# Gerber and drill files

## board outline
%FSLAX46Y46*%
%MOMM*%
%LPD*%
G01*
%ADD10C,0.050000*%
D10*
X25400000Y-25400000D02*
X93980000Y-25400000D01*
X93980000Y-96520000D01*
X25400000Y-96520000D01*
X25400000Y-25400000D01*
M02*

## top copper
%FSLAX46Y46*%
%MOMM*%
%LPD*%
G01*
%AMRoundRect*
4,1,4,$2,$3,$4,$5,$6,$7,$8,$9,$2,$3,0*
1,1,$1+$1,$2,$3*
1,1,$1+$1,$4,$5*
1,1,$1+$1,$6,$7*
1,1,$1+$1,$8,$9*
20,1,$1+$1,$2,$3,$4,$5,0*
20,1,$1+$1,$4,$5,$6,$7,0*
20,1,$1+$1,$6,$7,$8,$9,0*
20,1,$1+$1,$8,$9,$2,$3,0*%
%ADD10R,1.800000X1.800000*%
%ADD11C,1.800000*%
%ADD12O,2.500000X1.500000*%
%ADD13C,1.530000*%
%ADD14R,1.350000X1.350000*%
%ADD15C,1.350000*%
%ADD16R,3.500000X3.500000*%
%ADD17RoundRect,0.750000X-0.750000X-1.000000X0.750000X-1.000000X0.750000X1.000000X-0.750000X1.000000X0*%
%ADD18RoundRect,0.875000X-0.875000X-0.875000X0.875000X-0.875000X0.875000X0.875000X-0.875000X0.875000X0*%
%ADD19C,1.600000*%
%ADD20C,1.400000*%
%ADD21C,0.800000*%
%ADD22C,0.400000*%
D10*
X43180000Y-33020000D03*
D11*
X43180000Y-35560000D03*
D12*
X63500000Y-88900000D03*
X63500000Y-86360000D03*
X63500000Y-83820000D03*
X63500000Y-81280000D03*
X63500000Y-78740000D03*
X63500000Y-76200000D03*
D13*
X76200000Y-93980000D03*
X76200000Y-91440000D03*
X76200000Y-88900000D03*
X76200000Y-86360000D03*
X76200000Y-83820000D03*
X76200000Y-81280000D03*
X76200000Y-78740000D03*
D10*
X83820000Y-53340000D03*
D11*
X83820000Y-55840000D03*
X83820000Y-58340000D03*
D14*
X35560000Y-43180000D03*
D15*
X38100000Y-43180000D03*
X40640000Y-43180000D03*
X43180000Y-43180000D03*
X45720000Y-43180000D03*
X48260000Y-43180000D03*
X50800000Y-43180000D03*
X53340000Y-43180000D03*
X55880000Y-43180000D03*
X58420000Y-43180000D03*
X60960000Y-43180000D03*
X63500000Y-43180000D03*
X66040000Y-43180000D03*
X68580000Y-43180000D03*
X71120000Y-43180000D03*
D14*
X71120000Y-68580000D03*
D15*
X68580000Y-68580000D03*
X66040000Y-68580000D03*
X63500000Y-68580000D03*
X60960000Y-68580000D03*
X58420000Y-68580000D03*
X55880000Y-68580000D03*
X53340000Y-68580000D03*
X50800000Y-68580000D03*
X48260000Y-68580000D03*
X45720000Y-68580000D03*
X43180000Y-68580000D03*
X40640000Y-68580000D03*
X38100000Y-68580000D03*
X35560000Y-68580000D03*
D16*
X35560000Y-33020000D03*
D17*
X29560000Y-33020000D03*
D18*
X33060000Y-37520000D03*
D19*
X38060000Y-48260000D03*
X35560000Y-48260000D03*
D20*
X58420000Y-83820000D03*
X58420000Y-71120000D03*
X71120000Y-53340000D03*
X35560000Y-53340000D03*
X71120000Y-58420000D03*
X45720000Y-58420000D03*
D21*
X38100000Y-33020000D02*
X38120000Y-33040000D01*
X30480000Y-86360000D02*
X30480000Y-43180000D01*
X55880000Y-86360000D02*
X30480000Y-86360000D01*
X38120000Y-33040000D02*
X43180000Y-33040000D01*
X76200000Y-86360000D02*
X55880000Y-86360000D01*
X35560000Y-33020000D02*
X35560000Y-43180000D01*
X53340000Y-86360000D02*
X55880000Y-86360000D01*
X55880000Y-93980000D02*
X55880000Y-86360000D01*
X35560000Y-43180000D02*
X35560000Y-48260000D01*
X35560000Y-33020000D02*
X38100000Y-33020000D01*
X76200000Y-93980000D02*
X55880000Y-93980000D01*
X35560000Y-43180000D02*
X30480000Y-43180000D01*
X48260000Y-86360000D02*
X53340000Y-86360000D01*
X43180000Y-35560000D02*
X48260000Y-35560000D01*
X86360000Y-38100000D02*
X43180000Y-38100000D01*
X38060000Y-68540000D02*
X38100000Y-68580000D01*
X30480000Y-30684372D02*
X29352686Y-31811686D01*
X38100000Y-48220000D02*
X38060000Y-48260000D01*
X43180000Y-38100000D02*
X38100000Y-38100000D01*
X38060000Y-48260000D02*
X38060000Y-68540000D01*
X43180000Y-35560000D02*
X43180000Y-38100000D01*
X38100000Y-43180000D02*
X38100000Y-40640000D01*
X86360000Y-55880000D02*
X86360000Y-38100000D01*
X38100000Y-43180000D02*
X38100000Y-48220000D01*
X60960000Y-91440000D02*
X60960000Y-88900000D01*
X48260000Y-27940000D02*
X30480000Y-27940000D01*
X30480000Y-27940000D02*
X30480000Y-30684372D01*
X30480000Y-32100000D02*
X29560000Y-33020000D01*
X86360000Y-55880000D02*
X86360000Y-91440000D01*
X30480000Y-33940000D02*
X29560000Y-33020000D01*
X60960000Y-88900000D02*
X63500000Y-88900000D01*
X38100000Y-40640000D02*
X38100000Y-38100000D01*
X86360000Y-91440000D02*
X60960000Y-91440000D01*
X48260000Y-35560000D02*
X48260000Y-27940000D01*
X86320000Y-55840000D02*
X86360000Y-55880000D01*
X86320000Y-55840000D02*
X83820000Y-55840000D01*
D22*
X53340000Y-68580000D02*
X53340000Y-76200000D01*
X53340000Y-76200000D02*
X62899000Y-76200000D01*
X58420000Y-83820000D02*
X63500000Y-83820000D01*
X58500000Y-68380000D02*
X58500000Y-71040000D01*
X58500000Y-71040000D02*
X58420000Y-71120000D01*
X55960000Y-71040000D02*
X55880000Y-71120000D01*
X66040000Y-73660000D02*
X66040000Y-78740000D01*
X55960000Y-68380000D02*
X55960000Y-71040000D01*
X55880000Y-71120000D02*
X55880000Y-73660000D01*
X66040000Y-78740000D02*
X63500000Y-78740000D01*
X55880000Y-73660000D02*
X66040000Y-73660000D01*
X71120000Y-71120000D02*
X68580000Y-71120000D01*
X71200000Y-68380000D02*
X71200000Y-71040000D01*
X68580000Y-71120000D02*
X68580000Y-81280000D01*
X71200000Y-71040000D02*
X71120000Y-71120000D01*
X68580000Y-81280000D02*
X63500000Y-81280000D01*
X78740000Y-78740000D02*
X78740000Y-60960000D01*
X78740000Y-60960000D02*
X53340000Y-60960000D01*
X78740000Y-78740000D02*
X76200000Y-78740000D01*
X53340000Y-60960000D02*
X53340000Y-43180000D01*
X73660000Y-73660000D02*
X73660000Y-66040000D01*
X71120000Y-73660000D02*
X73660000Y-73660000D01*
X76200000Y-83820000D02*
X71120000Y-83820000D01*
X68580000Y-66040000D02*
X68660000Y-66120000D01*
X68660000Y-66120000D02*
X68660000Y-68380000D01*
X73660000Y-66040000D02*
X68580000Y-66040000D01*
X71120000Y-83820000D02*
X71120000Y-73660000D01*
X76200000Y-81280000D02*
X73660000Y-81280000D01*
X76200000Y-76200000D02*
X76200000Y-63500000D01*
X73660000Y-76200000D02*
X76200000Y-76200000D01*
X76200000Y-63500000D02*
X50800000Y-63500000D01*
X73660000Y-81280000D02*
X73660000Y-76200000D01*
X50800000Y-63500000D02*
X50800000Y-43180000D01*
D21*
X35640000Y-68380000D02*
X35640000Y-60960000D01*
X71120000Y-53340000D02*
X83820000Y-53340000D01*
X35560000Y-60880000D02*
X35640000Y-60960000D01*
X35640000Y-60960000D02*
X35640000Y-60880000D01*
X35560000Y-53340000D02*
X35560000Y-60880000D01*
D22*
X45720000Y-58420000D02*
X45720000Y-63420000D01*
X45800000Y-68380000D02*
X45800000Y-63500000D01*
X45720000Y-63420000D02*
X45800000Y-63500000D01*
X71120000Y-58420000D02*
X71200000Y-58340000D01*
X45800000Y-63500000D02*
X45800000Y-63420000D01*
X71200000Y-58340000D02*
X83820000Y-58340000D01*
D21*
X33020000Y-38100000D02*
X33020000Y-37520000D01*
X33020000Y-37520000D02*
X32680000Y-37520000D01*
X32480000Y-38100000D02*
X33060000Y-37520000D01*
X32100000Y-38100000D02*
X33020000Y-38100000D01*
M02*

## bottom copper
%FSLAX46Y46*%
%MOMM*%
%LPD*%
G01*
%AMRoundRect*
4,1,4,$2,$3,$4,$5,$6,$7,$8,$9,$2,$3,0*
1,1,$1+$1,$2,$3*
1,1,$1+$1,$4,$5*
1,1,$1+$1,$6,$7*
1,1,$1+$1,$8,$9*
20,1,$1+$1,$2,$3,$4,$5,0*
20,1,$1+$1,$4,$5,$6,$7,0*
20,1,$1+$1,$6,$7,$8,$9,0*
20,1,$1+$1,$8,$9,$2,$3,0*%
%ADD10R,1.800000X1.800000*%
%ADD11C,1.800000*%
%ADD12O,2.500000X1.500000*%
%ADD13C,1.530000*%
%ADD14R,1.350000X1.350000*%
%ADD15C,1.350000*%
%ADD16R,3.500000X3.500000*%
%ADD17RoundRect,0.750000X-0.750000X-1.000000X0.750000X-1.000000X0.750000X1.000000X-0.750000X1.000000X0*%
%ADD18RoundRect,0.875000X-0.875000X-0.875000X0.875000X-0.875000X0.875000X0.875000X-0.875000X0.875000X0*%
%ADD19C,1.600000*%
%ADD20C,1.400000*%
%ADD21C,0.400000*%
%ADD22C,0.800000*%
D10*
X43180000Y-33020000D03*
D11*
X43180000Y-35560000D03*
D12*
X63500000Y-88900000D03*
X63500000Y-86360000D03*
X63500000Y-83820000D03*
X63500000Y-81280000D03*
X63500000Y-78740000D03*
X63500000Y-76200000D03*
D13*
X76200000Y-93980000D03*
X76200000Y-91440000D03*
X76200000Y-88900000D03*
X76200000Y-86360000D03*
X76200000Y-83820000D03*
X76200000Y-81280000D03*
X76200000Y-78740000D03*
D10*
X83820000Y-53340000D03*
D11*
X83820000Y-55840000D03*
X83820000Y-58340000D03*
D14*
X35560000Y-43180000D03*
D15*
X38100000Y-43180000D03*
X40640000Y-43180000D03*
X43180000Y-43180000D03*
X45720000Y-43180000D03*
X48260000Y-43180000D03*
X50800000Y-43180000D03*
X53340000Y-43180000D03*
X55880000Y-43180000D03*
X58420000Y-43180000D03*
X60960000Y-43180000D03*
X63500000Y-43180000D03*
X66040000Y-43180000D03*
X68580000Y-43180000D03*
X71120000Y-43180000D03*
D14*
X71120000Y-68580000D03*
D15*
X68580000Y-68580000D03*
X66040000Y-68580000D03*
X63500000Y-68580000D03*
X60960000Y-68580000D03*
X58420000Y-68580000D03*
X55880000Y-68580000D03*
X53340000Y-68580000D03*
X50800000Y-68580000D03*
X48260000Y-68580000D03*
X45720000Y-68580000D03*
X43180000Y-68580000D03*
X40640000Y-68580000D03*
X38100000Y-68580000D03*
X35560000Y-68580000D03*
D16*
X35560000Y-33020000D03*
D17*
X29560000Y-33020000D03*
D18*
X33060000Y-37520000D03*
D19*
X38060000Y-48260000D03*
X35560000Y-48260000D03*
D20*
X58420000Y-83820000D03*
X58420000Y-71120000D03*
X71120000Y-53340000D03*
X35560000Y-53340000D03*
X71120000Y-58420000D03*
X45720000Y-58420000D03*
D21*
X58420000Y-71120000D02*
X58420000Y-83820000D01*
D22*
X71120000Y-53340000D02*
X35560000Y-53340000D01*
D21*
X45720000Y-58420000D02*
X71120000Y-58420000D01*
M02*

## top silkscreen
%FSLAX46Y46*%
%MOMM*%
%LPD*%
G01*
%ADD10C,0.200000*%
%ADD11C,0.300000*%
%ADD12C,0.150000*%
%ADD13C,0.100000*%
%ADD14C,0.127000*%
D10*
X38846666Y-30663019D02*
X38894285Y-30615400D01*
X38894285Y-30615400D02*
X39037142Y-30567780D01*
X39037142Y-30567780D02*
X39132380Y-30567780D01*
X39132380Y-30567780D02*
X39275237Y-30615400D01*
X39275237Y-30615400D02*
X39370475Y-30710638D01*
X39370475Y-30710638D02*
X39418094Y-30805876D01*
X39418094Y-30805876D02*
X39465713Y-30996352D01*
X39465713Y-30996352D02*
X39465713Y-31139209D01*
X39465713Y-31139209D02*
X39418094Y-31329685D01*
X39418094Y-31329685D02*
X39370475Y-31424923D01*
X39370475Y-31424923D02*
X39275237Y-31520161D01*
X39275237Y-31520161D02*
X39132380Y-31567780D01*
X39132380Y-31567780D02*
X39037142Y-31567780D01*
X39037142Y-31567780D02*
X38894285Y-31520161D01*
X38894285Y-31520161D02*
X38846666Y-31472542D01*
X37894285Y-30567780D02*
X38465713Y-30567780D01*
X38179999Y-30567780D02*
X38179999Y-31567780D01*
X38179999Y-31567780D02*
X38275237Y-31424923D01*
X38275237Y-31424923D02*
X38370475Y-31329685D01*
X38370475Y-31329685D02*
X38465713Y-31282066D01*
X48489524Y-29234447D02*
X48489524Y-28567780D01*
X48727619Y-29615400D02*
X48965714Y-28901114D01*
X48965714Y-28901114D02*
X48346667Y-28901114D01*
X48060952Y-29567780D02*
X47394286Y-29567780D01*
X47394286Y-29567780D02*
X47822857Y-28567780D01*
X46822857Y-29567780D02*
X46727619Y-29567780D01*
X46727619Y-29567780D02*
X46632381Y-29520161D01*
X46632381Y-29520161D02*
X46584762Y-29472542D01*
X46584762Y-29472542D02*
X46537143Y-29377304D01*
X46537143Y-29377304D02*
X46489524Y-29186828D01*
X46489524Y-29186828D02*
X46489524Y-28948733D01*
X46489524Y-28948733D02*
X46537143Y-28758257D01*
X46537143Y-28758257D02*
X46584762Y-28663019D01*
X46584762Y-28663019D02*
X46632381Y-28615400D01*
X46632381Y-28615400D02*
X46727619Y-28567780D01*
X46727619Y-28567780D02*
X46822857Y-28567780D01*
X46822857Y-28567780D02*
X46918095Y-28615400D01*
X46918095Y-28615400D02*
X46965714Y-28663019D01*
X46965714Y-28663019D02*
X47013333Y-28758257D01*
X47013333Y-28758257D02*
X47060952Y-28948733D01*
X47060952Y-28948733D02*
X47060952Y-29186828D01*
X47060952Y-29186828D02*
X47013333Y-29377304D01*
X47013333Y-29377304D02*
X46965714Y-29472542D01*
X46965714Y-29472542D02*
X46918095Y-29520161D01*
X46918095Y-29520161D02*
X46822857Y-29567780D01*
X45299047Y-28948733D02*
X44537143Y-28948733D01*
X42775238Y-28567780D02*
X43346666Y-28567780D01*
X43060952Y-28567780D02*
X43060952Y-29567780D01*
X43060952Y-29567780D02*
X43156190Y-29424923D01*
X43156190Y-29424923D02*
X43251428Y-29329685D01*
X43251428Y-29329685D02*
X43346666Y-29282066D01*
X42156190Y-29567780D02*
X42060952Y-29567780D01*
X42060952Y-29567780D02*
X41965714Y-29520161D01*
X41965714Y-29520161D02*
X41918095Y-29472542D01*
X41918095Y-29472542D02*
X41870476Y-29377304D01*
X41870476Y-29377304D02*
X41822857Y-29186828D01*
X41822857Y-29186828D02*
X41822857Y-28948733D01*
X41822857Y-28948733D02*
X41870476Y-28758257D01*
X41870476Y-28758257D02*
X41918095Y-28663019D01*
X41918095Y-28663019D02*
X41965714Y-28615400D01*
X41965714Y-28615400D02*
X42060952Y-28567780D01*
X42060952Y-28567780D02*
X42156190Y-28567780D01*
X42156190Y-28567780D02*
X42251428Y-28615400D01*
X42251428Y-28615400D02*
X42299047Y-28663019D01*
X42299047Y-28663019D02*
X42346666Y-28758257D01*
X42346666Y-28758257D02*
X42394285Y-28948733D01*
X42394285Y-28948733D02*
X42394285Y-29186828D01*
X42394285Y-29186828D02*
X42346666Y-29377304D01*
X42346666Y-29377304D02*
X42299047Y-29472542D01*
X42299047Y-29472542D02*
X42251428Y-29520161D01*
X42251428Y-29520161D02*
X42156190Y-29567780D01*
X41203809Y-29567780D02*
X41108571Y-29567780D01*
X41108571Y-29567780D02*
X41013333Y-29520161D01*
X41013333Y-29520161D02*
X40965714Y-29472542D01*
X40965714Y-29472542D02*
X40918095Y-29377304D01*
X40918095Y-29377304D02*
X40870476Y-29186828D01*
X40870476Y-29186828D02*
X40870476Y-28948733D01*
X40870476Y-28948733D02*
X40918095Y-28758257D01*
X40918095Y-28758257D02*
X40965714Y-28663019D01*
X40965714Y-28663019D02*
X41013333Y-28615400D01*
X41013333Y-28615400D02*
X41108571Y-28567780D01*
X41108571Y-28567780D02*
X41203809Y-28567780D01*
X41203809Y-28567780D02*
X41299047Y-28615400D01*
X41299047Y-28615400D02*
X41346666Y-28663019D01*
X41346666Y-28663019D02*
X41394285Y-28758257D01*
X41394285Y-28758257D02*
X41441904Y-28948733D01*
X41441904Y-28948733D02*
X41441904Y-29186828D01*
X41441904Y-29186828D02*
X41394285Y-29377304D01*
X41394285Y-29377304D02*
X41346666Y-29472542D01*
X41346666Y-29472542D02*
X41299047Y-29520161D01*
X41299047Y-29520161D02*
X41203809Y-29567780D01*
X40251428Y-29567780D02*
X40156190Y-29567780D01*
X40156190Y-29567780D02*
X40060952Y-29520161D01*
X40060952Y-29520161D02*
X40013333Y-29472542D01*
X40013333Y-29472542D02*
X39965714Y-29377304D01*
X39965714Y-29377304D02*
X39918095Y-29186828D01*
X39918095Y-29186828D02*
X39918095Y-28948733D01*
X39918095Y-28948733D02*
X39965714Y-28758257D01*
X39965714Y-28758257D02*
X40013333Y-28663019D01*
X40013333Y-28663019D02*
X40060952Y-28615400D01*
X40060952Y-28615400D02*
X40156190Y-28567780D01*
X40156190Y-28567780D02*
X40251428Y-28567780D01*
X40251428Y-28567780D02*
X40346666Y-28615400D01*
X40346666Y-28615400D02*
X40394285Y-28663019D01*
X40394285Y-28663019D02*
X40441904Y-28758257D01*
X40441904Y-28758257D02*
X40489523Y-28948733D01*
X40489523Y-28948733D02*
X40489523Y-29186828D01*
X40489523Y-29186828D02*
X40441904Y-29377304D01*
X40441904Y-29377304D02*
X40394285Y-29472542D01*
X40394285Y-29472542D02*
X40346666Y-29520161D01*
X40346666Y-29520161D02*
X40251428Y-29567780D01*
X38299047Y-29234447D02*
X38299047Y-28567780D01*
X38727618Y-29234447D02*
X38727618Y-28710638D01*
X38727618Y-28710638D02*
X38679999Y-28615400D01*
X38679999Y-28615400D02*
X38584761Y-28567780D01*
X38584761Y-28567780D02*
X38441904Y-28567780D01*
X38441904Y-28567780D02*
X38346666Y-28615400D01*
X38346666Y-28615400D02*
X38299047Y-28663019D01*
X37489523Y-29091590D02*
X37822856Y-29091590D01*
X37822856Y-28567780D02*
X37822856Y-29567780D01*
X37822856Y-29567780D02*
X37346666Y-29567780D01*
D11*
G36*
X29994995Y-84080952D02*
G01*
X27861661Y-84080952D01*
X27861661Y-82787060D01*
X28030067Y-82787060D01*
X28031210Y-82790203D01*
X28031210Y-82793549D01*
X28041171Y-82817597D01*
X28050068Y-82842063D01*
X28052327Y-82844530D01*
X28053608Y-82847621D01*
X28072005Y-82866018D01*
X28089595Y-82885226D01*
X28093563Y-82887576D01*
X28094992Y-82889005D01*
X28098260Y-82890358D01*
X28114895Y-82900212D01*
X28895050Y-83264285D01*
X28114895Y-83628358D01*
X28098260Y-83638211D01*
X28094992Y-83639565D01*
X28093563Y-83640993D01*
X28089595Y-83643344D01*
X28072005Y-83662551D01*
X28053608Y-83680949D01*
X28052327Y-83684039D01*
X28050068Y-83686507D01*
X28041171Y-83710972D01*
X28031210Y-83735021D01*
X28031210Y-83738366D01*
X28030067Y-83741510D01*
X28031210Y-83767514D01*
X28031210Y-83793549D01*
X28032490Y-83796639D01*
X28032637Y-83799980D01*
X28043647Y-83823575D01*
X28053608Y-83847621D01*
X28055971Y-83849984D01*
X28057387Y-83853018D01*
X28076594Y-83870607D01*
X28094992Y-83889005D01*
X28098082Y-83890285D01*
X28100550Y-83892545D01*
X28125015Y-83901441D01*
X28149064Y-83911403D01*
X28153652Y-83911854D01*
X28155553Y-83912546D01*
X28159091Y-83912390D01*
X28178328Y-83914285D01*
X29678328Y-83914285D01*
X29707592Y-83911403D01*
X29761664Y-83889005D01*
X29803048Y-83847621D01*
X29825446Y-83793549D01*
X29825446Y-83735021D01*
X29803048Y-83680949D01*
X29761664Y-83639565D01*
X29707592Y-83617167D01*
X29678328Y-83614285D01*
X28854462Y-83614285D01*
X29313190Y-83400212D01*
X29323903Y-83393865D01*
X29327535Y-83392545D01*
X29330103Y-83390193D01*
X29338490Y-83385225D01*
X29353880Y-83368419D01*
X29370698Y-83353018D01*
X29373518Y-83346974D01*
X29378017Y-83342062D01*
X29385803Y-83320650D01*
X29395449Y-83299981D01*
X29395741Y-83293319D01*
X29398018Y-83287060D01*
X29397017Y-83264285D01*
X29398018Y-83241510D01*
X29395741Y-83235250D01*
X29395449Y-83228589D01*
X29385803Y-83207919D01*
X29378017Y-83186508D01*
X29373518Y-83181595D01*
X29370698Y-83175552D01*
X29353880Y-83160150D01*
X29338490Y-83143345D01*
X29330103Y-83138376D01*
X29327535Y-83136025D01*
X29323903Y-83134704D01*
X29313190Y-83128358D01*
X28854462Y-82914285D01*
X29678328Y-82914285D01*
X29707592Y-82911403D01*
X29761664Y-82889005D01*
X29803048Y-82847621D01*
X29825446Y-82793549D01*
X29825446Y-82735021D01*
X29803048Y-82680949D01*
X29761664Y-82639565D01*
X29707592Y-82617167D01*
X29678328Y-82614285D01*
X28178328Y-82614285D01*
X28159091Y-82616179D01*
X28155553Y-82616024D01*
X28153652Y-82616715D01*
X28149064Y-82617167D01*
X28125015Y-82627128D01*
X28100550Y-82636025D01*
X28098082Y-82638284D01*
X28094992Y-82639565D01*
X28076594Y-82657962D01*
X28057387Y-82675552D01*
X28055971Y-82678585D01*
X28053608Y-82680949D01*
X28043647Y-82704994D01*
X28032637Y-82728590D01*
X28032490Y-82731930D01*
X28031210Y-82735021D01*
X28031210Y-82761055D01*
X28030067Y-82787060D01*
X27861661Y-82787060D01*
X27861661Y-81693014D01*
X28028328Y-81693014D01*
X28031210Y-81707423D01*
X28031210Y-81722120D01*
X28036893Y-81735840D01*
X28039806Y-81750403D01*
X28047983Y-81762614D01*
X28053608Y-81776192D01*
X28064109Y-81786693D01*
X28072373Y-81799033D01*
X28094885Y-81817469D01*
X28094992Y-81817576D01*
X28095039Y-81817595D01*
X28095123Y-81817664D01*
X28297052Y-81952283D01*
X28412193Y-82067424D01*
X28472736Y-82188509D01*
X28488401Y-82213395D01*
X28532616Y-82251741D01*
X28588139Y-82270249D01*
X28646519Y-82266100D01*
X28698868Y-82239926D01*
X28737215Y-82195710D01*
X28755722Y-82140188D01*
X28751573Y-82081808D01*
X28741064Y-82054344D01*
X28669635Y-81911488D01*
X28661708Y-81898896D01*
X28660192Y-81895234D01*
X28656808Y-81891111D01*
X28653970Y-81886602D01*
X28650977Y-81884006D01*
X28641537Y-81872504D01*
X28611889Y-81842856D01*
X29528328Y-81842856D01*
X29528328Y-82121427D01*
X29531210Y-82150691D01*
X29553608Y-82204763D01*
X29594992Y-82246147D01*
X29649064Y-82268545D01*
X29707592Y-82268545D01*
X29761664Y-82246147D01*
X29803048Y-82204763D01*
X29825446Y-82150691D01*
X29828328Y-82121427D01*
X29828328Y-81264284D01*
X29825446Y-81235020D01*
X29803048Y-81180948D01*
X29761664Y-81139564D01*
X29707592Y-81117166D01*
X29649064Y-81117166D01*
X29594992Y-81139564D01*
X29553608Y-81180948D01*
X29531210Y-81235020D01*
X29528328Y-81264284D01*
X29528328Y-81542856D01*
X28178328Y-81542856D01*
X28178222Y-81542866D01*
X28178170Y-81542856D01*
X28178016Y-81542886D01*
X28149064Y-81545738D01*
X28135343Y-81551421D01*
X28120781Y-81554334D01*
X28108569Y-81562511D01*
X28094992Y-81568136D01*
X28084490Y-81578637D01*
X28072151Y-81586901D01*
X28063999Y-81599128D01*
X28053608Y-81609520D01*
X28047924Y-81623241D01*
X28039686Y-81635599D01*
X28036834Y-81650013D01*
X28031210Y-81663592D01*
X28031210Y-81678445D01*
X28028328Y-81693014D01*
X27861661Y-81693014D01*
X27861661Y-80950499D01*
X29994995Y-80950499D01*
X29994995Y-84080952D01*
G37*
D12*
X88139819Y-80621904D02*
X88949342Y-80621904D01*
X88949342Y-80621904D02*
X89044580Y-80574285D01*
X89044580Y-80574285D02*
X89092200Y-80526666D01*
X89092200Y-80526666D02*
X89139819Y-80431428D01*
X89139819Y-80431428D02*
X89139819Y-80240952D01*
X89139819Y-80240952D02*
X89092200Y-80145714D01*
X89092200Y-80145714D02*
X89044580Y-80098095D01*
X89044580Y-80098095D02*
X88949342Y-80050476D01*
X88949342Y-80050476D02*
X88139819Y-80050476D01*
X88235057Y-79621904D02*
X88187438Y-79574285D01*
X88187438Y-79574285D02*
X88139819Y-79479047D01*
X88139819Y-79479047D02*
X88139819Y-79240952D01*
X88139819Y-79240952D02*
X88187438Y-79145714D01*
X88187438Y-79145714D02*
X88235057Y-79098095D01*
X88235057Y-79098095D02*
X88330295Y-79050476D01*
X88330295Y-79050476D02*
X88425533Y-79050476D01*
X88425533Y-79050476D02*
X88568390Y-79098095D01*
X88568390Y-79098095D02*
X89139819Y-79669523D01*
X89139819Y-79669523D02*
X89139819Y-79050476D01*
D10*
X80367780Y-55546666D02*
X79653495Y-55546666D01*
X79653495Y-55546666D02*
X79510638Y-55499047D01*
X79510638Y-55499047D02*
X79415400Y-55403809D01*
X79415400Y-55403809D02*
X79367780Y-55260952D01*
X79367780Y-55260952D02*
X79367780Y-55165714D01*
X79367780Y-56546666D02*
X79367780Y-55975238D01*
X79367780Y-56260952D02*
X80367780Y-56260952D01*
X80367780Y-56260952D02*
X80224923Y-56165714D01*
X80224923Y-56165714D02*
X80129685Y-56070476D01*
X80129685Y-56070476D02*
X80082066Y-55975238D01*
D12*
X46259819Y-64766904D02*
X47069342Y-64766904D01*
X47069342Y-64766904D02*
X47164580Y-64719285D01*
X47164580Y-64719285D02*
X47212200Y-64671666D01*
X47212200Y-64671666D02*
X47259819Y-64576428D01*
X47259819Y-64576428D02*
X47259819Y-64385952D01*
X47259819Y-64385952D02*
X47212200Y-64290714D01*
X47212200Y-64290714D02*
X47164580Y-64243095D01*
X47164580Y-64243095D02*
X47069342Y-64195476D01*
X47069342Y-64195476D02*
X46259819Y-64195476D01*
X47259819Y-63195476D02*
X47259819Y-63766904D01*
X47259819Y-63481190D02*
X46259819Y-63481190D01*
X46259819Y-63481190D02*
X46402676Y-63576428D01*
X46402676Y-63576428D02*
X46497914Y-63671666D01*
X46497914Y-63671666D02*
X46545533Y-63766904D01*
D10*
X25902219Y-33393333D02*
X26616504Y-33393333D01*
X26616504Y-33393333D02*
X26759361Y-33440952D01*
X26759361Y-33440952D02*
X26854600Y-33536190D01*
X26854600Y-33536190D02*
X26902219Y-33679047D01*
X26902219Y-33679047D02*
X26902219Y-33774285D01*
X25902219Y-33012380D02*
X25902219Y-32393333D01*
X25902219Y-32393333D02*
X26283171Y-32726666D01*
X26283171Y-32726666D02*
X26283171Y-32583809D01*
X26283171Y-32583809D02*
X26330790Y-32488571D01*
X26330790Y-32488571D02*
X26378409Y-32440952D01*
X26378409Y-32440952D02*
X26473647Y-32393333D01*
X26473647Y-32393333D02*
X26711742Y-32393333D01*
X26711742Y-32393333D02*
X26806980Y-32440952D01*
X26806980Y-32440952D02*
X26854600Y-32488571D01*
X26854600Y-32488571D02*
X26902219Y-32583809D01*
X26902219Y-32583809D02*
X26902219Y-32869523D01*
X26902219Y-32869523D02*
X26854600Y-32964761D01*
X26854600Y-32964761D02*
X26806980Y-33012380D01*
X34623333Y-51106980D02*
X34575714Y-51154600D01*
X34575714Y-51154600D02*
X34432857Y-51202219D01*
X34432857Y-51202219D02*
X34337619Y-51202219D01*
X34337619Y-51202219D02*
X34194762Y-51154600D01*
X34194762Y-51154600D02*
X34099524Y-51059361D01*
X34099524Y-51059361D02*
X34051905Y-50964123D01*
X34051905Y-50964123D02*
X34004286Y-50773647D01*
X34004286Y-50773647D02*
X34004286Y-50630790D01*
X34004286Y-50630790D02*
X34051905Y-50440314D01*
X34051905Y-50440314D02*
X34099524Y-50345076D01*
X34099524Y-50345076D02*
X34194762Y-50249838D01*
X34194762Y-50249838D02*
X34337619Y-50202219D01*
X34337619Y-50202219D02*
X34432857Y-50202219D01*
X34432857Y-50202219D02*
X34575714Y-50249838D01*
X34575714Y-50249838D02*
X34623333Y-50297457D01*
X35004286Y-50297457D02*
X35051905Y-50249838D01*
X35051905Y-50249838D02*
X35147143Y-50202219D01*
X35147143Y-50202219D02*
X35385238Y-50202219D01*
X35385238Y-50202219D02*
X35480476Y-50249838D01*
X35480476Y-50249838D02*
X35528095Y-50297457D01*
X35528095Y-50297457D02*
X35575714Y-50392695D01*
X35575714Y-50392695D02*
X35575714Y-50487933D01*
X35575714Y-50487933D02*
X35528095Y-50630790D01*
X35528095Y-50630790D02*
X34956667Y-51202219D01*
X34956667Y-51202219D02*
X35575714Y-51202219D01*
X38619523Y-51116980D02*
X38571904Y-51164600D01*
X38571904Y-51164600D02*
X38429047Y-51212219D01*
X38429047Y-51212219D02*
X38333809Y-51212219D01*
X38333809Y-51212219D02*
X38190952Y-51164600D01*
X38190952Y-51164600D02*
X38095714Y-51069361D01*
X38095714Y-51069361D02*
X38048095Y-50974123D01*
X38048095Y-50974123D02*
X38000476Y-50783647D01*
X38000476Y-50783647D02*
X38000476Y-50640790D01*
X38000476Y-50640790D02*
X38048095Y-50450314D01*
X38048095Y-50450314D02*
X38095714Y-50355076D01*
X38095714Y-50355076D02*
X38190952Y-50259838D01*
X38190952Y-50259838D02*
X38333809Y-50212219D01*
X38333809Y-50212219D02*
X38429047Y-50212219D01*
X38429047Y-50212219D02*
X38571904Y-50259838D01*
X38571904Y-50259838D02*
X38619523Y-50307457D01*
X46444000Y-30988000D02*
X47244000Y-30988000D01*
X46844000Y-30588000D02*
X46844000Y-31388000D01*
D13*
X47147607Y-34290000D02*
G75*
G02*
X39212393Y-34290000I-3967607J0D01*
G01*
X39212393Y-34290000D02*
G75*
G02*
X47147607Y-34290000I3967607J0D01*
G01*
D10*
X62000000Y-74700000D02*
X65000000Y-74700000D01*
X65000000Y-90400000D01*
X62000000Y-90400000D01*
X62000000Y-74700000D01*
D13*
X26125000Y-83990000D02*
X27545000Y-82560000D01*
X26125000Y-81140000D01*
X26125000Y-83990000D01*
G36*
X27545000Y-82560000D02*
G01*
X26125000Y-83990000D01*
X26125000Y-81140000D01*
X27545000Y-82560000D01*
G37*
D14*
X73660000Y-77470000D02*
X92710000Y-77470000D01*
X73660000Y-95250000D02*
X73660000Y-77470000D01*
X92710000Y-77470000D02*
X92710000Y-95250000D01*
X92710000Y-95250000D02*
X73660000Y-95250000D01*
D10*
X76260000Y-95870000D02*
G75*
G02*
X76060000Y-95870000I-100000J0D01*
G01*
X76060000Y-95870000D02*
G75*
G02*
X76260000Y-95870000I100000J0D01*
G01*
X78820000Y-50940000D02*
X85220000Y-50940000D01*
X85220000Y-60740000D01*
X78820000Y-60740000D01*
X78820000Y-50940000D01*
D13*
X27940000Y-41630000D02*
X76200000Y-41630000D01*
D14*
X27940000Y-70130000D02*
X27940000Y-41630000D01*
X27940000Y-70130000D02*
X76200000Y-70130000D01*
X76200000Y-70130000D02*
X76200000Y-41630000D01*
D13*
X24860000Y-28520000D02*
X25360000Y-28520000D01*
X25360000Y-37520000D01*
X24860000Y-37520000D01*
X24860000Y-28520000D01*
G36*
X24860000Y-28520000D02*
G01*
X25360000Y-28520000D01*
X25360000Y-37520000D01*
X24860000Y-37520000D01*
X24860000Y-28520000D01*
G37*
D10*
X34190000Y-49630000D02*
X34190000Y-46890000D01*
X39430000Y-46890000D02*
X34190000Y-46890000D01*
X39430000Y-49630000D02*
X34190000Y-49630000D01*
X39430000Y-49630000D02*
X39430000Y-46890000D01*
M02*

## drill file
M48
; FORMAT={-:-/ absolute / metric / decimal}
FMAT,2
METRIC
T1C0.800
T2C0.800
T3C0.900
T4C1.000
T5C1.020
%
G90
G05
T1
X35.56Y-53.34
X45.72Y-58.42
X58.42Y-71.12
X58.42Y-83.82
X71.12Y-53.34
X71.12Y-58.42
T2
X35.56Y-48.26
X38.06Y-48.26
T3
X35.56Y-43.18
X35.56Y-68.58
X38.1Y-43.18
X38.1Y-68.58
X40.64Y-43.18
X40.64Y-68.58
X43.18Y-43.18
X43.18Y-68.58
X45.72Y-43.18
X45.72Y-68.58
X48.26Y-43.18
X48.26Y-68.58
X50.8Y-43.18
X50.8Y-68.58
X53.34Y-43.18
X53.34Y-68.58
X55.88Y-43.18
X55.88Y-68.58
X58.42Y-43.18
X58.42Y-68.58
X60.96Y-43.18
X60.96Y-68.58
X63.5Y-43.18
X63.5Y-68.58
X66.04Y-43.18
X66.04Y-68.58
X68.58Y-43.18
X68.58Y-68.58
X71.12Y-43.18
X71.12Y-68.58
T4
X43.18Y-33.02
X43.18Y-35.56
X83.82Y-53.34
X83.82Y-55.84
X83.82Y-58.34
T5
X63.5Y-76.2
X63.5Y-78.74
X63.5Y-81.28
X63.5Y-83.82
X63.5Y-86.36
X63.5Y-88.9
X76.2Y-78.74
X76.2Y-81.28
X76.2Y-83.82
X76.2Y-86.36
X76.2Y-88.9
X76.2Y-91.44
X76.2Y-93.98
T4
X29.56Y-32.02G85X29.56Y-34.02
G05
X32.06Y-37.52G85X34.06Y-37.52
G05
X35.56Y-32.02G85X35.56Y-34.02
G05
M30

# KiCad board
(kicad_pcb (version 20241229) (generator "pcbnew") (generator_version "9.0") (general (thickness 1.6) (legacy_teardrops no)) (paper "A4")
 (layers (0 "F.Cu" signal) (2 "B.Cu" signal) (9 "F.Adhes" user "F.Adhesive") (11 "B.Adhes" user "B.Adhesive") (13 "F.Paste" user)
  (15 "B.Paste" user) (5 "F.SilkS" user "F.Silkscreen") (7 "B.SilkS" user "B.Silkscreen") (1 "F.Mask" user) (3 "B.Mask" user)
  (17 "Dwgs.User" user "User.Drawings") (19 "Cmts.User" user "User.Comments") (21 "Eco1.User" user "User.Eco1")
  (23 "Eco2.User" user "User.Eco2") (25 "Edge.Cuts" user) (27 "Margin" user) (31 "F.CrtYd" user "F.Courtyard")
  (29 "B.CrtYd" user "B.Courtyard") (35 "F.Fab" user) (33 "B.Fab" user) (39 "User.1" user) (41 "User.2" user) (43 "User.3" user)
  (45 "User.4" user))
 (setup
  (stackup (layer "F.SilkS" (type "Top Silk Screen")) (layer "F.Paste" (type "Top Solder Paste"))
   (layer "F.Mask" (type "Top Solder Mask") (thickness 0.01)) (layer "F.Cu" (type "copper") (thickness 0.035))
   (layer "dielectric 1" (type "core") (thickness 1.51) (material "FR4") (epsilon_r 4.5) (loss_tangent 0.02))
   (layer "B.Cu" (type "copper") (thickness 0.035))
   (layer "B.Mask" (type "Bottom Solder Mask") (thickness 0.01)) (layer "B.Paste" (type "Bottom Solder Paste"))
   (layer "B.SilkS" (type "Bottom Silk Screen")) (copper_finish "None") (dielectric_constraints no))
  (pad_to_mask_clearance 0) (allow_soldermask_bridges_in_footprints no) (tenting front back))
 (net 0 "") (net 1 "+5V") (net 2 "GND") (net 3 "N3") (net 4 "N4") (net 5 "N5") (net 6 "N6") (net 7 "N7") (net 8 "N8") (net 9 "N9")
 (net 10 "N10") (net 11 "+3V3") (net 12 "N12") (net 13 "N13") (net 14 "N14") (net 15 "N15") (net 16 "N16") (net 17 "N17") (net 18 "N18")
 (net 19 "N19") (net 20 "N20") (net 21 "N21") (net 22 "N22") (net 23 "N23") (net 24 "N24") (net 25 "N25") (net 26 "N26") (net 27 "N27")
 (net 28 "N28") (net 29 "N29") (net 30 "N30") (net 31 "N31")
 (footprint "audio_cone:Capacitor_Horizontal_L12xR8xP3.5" (layer "F.Cu") (at 43.18 33.02 -90)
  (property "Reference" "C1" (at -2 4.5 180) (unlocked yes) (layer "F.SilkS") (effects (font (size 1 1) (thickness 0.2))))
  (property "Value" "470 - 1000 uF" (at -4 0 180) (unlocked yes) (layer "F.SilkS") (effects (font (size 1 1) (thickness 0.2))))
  (fp_line (start -2.032 -3.264) (end -2.032 -4.064) (stroke (width 0.2) (type solid)) (layer "F.SilkS"))
  (fp_line (start -2.432 -3.664) (end -1.632 -3.664) (stroke (width 0.2) (type solid)) (layer "F.SilkS"))
  (fp_circle (center 1.27 0) (end 4.318 2.54) (stroke (width 0.1) (type default)) (fill no) (layer "F.SilkS"))
  (pad "1" thru_hole rect (at 0 0 90) (size 1.8 1.8) (drill 1) (layers "*.Cu" "*.Mask") (remove_unused_layers no) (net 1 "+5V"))
  (pad "2" thru_hole circle (at 2.54 0 90) (size 1.8 1.8) (drill 1) (layers "*.Cu" "*.Mask") (remove_unused_layers no) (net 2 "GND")))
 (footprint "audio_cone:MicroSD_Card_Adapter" (layer "F.Cu") (at 63.5 88.9 90)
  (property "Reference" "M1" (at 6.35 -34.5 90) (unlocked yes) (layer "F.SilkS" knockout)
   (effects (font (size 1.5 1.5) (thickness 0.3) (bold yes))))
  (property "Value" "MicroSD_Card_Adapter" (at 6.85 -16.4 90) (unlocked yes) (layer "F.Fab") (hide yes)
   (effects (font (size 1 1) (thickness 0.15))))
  (fp_rect (start -1.5 -1.5) (end 14.2 1.5) (stroke (width 0.2) (type solid)) (fill no) (layer "F.SilkS"))
  (fp_poly (pts (xy 4.91 -37.375) (xy 6.34 -35.955) (xy 7.76 -37.375)) (stroke (width 0.1) (type solid)) (fill yes) (layer "F.SilkS"))
  (pad "1" thru_hole oval (at 0 0 90) (size 1.5 2.5) (drill 1.02) (layers "*.Cu" "*.Mask") (remove_unused_layers no) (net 2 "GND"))
  (pad "2" thru_hole oval (at 2.54 0 90) (size 1.5 2.5) (drill 1.02) (layers "*.Cu" "*.Mask") (remove_unused_layers no) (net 1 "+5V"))
  (pad "3" thru_hole oval (at 5.08 0 90) (size 1.5 2.5) (drill 1.02) (layers "*.Cu" "*.Mask") (remove_unused_layers no) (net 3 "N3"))
  (pad "4" thru_hole oval (at 7.62 0 90) (size 1.5 2.5) (drill 1.02) (layers "*.Cu" "*.Mask") (remove_unused_layers no) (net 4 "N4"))
  (pad "5" thru_hole oval (at 10.16 0 90) (size 1.5 2.5) (drill 1.02) (layers "*.Cu" "*.Mask") (remove_unused_layers no) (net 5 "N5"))
  (pad "6" thru_hole oval (at 12.7 0 90) (size 1.5 2.5) (drill 1.02) (layers "*.Cu" "*.Mask") (remove_unused_layers no) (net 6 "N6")))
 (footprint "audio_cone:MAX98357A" (layer "F.Cu") (at 83.185 86.36 -90)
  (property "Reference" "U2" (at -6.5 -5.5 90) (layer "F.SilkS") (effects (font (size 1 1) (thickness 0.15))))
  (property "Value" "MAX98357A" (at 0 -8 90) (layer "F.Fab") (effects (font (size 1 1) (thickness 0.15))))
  (fp_line (start -8.89 9.525) (end -8.89 -9.525) (stroke (width 0.127) (type solid)) (layer "F.SilkS"))
  (fp_line (start 8.89 9.525) (end -8.89 9.525) (stroke (width 0.127) (type solid)) (layer "F.SilkS"))
  (fp_line (start -8.89 -9.525) (end 8.89 -9.525) (stroke (width 0.127) (type solid)) (layer "F.SilkS"))
  (fp_line (start 8.89 -9.525) (end 8.89 9.525) (stroke (width 0.127) (type solid)) (layer "F.SilkS"))
  (fp_circle (center 9.51 7.025) (end 9.61 7.025) (stroke (width 0.2) (type solid)) (fill no) (layer "F.SilkS"))
  (pad "JP1_1" thru_hole circle (at 7.62 6.985 270) (size 1.53 1.53) (drill 1.02) (layers "*.Cu" "*.Mask") (remove_unused_layers no)
   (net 1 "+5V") (solder_mask_margin 0.102))
  (pad "JP1_2" thru_hole circle (at 5.08 6.985 270) (size 1.53 1.53) (drill 1.02) (layers "*.Cu" "*.Mask") (remove_unused_layers no)
   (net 2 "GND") (solder_mask_margin 0.102))
  (pad "JP1_3" thru_hole circle (at 2.54 6.985 270) (size 1.53 1.53) (drill 1.02) (layers "*.Cu" "*.Mask") (remove_unused_layers no)
   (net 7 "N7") (solder_mask_margin 0.102))
  (pad "JP1_4" thru_hole circle (at 0 6.985 270) (size 1.53 1.53) (drill 1.02) (layers "*.Cu" "*.Mask") (remove_unused_layers no)
   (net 1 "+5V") (solder_mask_margin 0.102))
  (pad "JP1_5" thru_hole circle (at -2.54 6.985 270) (size 1.53 1.53) (drill 1.02) (layers "*.Cu" "*.Mask") (remove_unused_layers no)
   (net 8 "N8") (solder_mask_margin 0.102))
  (pad "JP1_6" thru_hole circle (at -5.08 6.985 270) (size 1.53 1.53) (drill 1.02) (layers "*.Cu" "*.Mask") (remove_unused_layers no)
   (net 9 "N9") (solder_mask_margin 0.102))
  (pad "JP1_7" thru_hole circle (at -7.62 6.985 270) (size 1.53 1.53) (drill 1.02) (layers "*.Cu" "*.Mask") (remove_unused_layers no)
   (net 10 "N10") (solder_mask_margin 0.102)))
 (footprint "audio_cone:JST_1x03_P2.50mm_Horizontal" (layer "F.Cu") (at 83.82 53.34 -90)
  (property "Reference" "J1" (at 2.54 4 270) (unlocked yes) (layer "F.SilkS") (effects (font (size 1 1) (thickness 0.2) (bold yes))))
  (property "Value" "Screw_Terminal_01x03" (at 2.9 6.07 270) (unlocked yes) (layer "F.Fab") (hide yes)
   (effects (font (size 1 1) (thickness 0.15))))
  (fp_rect (start 7.4 5) (end -2.4 -1.4) (stroke (width 0.2) (type solid)) (fill no) (layer "F.SilkS"))
  (pad "1" thru_hole rect (at 0 0 90) (size 1.8 1.8) (drill 1) (layers "*.Cu" "*.Mask") (remove_unused_layers no) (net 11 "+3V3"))
  (pad "2" thru_hole circle (at 2.5 0 90) (size 1.8 1.8) (drill 1) (layers "*.Cu" "*.Mask") (remove_unused_layers no) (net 2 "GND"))
  (pad "3" thru_hole circle (at 5 0 90) (size 1.8 1.8) (drill 1) (layers "*.Cu" "*.Mask") (remove_unused_layers no) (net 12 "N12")))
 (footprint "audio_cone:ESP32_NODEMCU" (layer "F.Cu") (at 76.2 55.88 -90)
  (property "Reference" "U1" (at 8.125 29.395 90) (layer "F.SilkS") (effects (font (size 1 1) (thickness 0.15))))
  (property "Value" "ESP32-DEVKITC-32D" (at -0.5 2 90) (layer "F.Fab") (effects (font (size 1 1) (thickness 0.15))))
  (fp_line (start -14.25 48.26) (end -14.25 0) (stroke (width 0.1) (type solid)) (layer "F.SilkS"))
  (fp_line (start 14.25 48.26) (end -14.25 48.26) (stroke (width 0.127) (type solid)) (layer "F.SilkS"))
  (fp_line (start 14.25 48.26) (end 14.25 0) (stroke (width 0.127) (type solid)) (layer "F.SilkS"))
  (fp_line (start 14.25 0) (end -14.25 0) (stroke (width 0.127) (type solid)) (layer "F.SilkS"))
  (pad "J1-01" thru_hole rect (at -12.7 40.64 90) (size 1.35 1.35) (drill 0.9) (layers "*.Cu" "*.Mask") (remove_unused_layers no)
   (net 1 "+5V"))
  (pad "J1-02" thru_hole circle (at -12.7 38.1 90) (size 1.35 1.35) (drill 0.9) (layers "*.Cu" "*.Mask") (remove_unused_layers no)
   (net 2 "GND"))
  (pad "J1-03" thru_hole circle (at -12.7 35.56 90) (size 1.35 1.35) (drill 0.9) (layers "*.Cu" "*.Mask") (remove_unused_layers no)
   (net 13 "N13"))
  (pad "J1-04" thru_hole circle (at -12.7 33.02 90) (size 1.35 1.35) (drill 0.9) (layers "*.Cu" "*.Mask") (remove_unused_layers no)
   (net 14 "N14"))
  (pad "J1-05" thru_hole circle (at -12.7 30.48 90) (size 1.35 1.35) (drill 0.9) (layers "*.Cu" "*.Mask") (remove_unused_layers no)
   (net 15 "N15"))
  (pad "J1-06" thru_hole circle (at -12.7 27.94 90) (size 1.35 1.35) (drill 0.9) (layers "*.Cu" "*.Mask") (remove_unused_layers no)
   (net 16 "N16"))
  (pad "J1-07" thru_hole circle (at -12.7 25.4 90) (size 1.35 1.35) (drill 0.9) (layers "*.Cu" "*.Mask") (remove_unused_layers no)
   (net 9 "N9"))
  (pad "J1-08" thru_hole circle (at -12.7 22.86 90) (size 1.35 1.35) (drill 0.9) (layers "*.Cu" "*.Mask") (remove_unused_layers no)
   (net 10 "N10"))
  (pad "J1-09" thru_hole circle (at -12.7 20.32 90) (size 1.35 1.35) (drill 0.9) (layers "*.Cu" "*.Mask") (remove_unused_layers no)
   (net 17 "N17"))
  (pad "J1-10" thru_hole circle (at -12.7 17.78 90) (size 1.35 1.35) (drill 0.9) (layers "*.Cu" "*.Mask") (remove_unused_layers no)
   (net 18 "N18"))
  (pad "J1-11" thru_hole circle (at -12.7 15.24 90) (size 1.35 1.35) (drill 0.9) (layers "*.Cu" "*.Mask") (remove_unused_layers no)
   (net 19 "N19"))
  (pad "J1-12" thru_hole circle (at -12.7 12.7 90) (size 1.35 1.35) (drill 0.9) (layers "*.Cu" "*.Mask") (remove_unused_layers no)
   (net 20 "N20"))
  (pad "J1-13" thru_hole circle (at -12.7 10.16 90) (size 1.35 1.35) (drill 0.9) (layers "*.Cu" "*.Mask") (remove_unused_layers no)
   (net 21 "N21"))
  (pad "J1-14" thru_hole circle (at -12.7 7.62 90) (size 1.35 1.35) (drill 0.9) (layers "*.Cu" "*.Mask") (remove_unused_layers no)
   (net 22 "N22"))
  (pad "J1-15" thru_hole circle (at -12.7 5.08 90) (size 1.35 1.35) (drill 0.9) (layers "*.Cu" "*.Mask") (remove_unused_layers no)
   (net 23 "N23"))
  (pad "J1-16" thru_hole rect (at 12.7 5.08 90) (size 1.35 1.35) (drill 0.9) (layers "*.Cu" "*.Mask") (remove_unused_layers no) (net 4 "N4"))
  (pad "J1-17" thru_hole circle (at 12.7 7.62 90) (size 1.35 1.35) (drill 0.9) (layers "*.Cu" "*.Mask") (remove_unused_layers no)
   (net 8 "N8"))
  (pad "J1-18" thru_hole circle (at 12.7 10.16 90) (size 1.35 1.35) (drill 0.9) (layers "*.Cu" "*.Mask") (remove_unused_layers no)
   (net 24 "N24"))
  (pad "J1-19" thru_hole circle (at 12.7 12.7 90) (size 1.35 1.35) (drill 0.9) (layers "*.Cu" "*.Mask") (remove_unused_layers no)
   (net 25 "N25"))
  (pad "J1-20" thru_hole circle (at 12.7 15.24 90) (size 1.35 1.35) (drill 0.9) (layers "*.Cu" "*.Mask") (remove_unused_layers no)
   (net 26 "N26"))
  (pad "J1-21" thru_hole circle (at 12.7 17.78 90) (size 1.35 1.35) (drill 0.9) (layers "*.Cu" "*.Mask") (remove_unused_layers no)
   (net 3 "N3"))
  (pad "J1-22" thru_hole circle (at 12.7 20.32 90) (size 1.35 1.35) (drill 0.9) (layers "*.Cu" "*.Mask") (remove_unused_layers no)
   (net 5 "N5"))
  (pad "J1-23" thru_hole circle (at 12.7 22.86 90) (size 1.35 1.35) (drill 0.9) (layers "*.Cu" "*.Mask") (remove_unused_layers no)
   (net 6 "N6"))
  (pad "J1-24" thru_hole circle (at 12.7 25.4 90) (size 1.35 1.35) (drill 0.9) (layers "*.Cu" "*.Mask") (remove_unused_layers no)
   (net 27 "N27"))
  (pad "J1-25" thru_hole circle (at 12.7 27.94 90) (size 1.35 1.35) (drill 0.9) (layers "*.Cu" "*.Mask") (remove_unused_layers no)
   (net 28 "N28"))
  (pad "J1-26" thru_hole circle (at 12.7 30.48 90) (size 1.35 1.35) (drill 0.9) (layers "*.Cu" "*.Mask") (remove_unused_layers no)
   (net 12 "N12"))
  (pad "J1-27" thru_hole circle (at 12.7 33.02 90) (size 1.35 1.35) (drill 0.9) (layers "*.Cu" "*.Mask") (remove_unused_layers no)
   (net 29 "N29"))
  (pad "J1-28" thru_hole circle (at 12.7 35.56 90) (size 1.35 1.35) (drill 0.9) (layers "*.Cu" "*.Mask") (remove_unused_layers no)
   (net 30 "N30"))
  (pad "J1-29" thru_hole circle (at 12.7 38.1 90) (size 1.35 1.35) (drill 0.9) (layers "*.Cu" "*.Mask") (remove_unused_layers no)
   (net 2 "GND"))
  (pad "J1-30" thru_hole circle (at 12.7 40.64 90) (size 1.35 1.35) (drill 0.9) (layers "*.Cu" "*.Mask") (remove_unused_layers no)
   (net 11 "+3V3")))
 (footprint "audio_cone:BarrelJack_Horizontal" (layer "F.Cu") (at 35.56 33.02 180)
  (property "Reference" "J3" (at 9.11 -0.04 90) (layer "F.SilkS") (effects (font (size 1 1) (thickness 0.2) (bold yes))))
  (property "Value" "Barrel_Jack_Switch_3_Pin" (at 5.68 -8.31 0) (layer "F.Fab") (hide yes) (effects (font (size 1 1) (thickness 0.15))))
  (fp_rect (start 10.2 -4.5) (end 10.7 4.5) (stroke (width 0.1) (type solid)) (fill yes) (layer "F.SilkS"))
  (pad "1" thru_hole rect (at 0 0) (size 3.5 3.5) (drill oval 1 3) (layers "*.Cu" "*.Mask") (remove_unused_layers no) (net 1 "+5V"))
  (pad "2" thru_hole roundrect (at 6 0) (size 3 3.5) (drill oval 1 3) (layers "*.Cu" "*.Mask") (remove_unused_layers no)
   (roundrect_rratio 0.25) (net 2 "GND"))
  (pad "3" thru_hole roundrect (at 2.5 -4.5) (size 3.5 3.5) (drill oval 3 1) (layers "*.Cu" "*.Mask") (remove_unused_layers no)
   (roundrect_rratio 0.25) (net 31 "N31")))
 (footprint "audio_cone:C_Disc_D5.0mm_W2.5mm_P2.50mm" (layer "F.Cu") (at 38.06 48.26 180)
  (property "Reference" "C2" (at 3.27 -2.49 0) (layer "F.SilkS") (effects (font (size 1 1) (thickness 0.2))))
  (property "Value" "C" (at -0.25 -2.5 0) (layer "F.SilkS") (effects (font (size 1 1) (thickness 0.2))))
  (fp_line (start 3.87 -1.37) (end 3.87 1.37) (stroke (width 0.2) (type solid)) (layer "F.SilkS"))
  (fp_line (start -1.37 1.37) (end 3.87 1.37) (stroke (width 0.2) (type solid)) (layer "F.SilkS"))
  (fp_line (start -1.37 -1.37) (end 3.87 -1.37) (stroke (width 0.2) (type solid)) (layer "F.SilkS"))
  (fp_line (start -1.37 -1.37) (end -1.37 1.37) (stroke (width 0.2) (type solid)) (layer "F.SilkS"))
  (pad "1" thru_hole circle (at 0 0 180) (size 1.6 1.6) (drill 0.8) (layers "*.Cu" "*.Mask") (remove_unused_layers no) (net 2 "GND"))
  (pad "2" thru_hole circle (at 2.5 0 180) (size 1.6 1.6) (drill 0.8) (layers "*.Cu" "*.Mask") (remove_unused_layers no) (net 1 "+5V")))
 (gr_rect (start 25.4 25.4) (end 93.98 96.52) (stroke (width 0.05) (type default)) (fill no) (layer "Edge.Cuts"))
 (segment (start 38.1 33.02) (end 38.12 33.04) (width 0.8) (layer "F.Cu") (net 1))
 (segment (start 30.48 86.36) (end 30.48 43.18) (width 0.8) (layer "F.Cu") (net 1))
 (segment (start 55.88 86.36) (end 30.48 86.36) (width 0.8) (layer "F.Cu") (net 1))
 (segment (start 38.12 33.04) (end 43.18 33.04) (width 0.8) (layer "F.Cu") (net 1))
 (segment (start 76.2 86.36) (end 55.88 86.36) (width 0.8) (layer "F.Cu") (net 1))
 (segment (start 35.56 33.02) (end 35.56 43.18) (width 0.8) (layer "F.Cu") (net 1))
 (segment (start 53.34 86.36) (end 55.88 86.36) (width 0.8) (layer "F.Cu") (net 1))
 (segment (start 55.88 93.98) (end 55.88 86.36) (width 0.8) (layer "F.Cu") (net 1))
 (segment (start 35.56 43.18) (end 35.56 48.26) (width 0.8) (layer "F.Cu") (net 1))
 (segment (start 35.56 33.02) (end 38.1 33.02) (width 0.8) (layer "F.Cu") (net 1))
 (segment (start 76.2 93.98) (end 55.88 93.98) (width 0.8) (layer "F.Cu") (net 1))
 (segment (start 35.56 43.18) (end 30.48 43.18) (width 0.8) (layer "F.Cu") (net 1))
 (segment (start 48.26 86.36) (end 53.34 86.36) (width 0.8) (layer "F.Cu") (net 1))
 (segment (start 43.18 35.56) (end 48.26 35.56) (width 0.8) (layer "F.Cu") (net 2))
 (segment (start 86.36 38.1) (end 43.18 38.1) (width 0.8) (layer "F.Cu") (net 2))
 (segment (start 38.06 68.54) (end 38.1 68.58) (width 0.8) (layer "F.Cu") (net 2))
 (segment (start 30.48 30.684372) (end 29.352686 31.811686) (width 0.8) (layer "F.Cu") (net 2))
 (segment (start 38.1 48.22) (end 38.06 48.26) (width 0.8) (layer "F.Cu") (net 2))
 (segment (start 43.18 38.1) (end 38.1 38.1) (width 0.8) (layer "F.Cu") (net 2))
 (segment (start 38.06 48.26) (end 38.06 68.54) (width 0.8) (layer "F.Cu") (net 2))
 (segment (start 43.18 35.56) (end 43.18 38.1) (width 0.8) (layer "F.Cu") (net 2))
 (segment (start 38.1 43.18) (end 38.1 40.64) (width 0.8) (layer "F.Cu") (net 2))
 (segment (start 86.36 55.88) (end 86.36 38.1) (width 0.8) (layer "F.Cu") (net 2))
 (segment (start 38.1 43.18) (end 38.1 48.22) (width 0.8) (layer "F.Cu") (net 2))
 (segment (start 60.96 91.44) (end 60.96 88.9) (width 0.8) (layer "F.Cu") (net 2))
 (segment (start 48.26 27.94) (end 30.48 27.94) (width 0.8) (layer "F.Cu") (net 2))
 (segment (start 30.48 27.94) (end 30.48 30.684372) (width 0.8) (layer "F.Cu") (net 2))
 (segment (start 30.48 32.1) (end 29.56 33.02) (width 0.8) (layer "F.Cu") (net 2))
 (segment (start 86.36 55.88) (end 86.36 91.44) (width 0.8) (layer "F.Cu") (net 2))
 (segment (start 30.48 33.94) (end 29.56 33.02) (width 0.8) (layer "F.Cu") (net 2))
 (segment (start 60.96 88.9) (end 63.5 88.9) (width 0.8) (layer "F.Cu") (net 2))
 (segment (start 38.1 40.64) (end 38.1 38.1) (width 0.8) (layer "F.Cu") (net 2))
 (segment (start 86.36 91.44) (end 60.96 91.44) (width 0.8) (layer "F.Cu") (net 2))
 (segment (start 48.26 35.56) (end 48.26 27.94) (width 0.8) (layer "F.Cu") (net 2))
 (segment (start 86.32 55.84) (end 86.36 55.88) (width 0.8) (layer "F.Cu") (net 2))
 (segment (start 86.32 55.84) (end 83.82 55.84) (width 0.8) (layer "F.Cu") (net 2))
 (segment (start 53.34 68.58) (end 53.34 76.2) (width 0.4) (layer "F.Cu") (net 6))
 (segment (start 53.34 76.2) (end 62.899 76.2) (width 0.4) (layer "F.Cu") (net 6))
 (segment (start 58.42 83.82) (end 63.5 83.82) (width 0.4) (layer "F.Cu") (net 3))
 (segment (start 58.5 68.38) (end 58.5 71.04) (width 0.4) (layer "F.Cu") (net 3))
 (segment (start 58.5 71.04) (end 58.42 71.12) (width 0.4) (layer "F.Cu") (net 3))
 (via (at 58.42 83.82) (size 1.4) (drill 0.8) (layers "F.Cu" "B.Cu") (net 3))
 (via (at 58.42 71.12) (size 1.4) (drill 0.8) (layers "F.Cu" "B.Cu") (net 3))
 (segment (start 58.42 71.12) (end 58.42 83.82) (width 0.4) (layer "B.Cu") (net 3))
 (segment (start 55.96 71.04) (end 55.88 71.12) (width 0.4) (layer "F.Cu") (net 5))
 (segment (start 66.04 73.66) (end 66.04 78.74) (width 0.4) (layer "F.Cu") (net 5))
 (segment (start 55.96 68.38) (end 55.96 71.04) (width 0.4) (layer "F.Cu") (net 5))
 (segment (start 55.88 71.12) (end 55.88 73.66) (width 0.4) (layer "F.Cu") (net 5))
 (segment (start 66.04 78.74) (end 63.5 78.74) (width 0.4) (layer "F.Cu") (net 5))
 (segment (start 55.88 73.66) (end 66.04 73.66) (width 0.4) (layer "F.Cu") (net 5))
 (segment (start 71.12 71.12) (end 68.58 71.12) (width 0.4) (layer "F.Cu") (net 4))
 (segment (start 71.2 68.38) (end 71.2 71.04) (width 0.4) (layer "F.Cu") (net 4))
 (segment (start 68.58 71.12) (end 68.58 81.28) (width 0.4) (layer "F.Cu") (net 4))
 (segment (start 71.2 71.04) (end 71.12 71.12) (width 0.4) (layer "F.Cu") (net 4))
 (segment (start 68.58 81.28) (end 63.5 81.28) (width 0.4) (layer "F.Cu") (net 4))
 (segment (start 78.74 78.74) (end 78.74 60.96) (width 0.4) (layer "F.Cu") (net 10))
 (segment (start 78.74 60.96) (end 53.34 60.96) (width 0.4) (layer "F.Cu") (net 10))
 (segment (start 78.74 78.74) (end 76.2 78.74) (width 0.4) (layer "F.Cu") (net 10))
 (segment (start 53.34 60.96) (end 53.34 43.18) (width 0.4) (layer "F.Cu") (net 10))
 (segment (start 73.66 73.66) (end 73.66 66.04) (width 0.4) (layer "F.Cu") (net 8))
 (segment (start 71.12 73.66) (end 73.66 73.66) (width 0.4) (layer "F.Cu") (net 8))
 (segment (start 76.2 83.82) (end 71.12 83.82) (width 0.4) (layer "F.Cu") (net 8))
 (segment (start 68.58 66.04) (end 68.66 66.12) (width 0.4) (layer "F.Cu") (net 8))
 (segment (start 68.66 66.12) (end 68.66 68.38) (width 0.4) (layer "F.Cu") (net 8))
 (segment (start 73.66 66.04) (end 68.58 66.04) (width 0.4) (layer "F.Cu") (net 8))
 (segment (start 71.12 83.82) (end 71.12 73.66) (width 0.4) (layer "F.Cu") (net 8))
 (segment (start 76.2 81.28) (end 73.66 81.28) (width 0.4) (layer "F.Cu") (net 9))
 (segment (start 76.2 76.2) (end 76.2 63.5) (width 0.4) (layer "F.Cu") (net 9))
 (segment (start 73.66 76.2) (end 76.2 76.2) (width 0.4) (layer "F.Cu") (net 9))
 (segment (start 76.2 63.5) (end 50.8 63.5) (width 0.4) (layer "F.Cu") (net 9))
 (segment (start 73.66 81.28) (end 73.66 76.2) (width 0.4) (layer "F.Cu") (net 9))
 (segment (start 50.8 63.5) (end 50.8 43.18) (width 0.4) (layer "F.Cu") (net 9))
 (segment (start 35.64 68.38) (end 35.64 60.96) (width 0.8) (layer "F.Cu") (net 11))
 (segment (start 71.12 53.34) (end 83.82 53.34) (width 0.8) (layer "F.Cu") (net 11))
 (segment (start 35.56 60.88) (end 35.64 60.96) (width 0.8) (layer "F.Cu") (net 11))
 (segment (start 35.64 60.96) (end 35.64 60.88) (width 0.8) (layer "F.Cu") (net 11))
 (segment (start 35.56 53.34) (end 35.56 60.88) (width 0.8) (layer "F.Cu") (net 11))
 (via (at 71.12 53.34) (size 1.4) (drill 0.8) (layers "F.Cu" "B.Cu") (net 11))
 (via (at 35.56 53.34) (size 1.4) (drill 0.8) (layers "F.Cu" "B.Cu") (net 11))
 (segment (start 71.12 53.34) (end 35.56 53.34) (width 0.8) (layer "B.Cu") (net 11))
 (segment (start 45.72 58.42) (end 45.72 63.42) (width 0.4) (layer "F.Cu") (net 12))
 (segment (start 45.8 68.38) (end 45.8 63.5) (width 0.4) (layer "F.Cu") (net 12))
 (segment (start 45.72 63.42) (end 45.8 63.5) (width 0.4) (layer "F.Cu") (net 12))
 (segment (start 71.12 58.42) (end 71.2 58.34) (width 0.4) (layer "F.Cu") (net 12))
 (segment (start 45.8 63.5) (end 45.8 63.42) (width 0.4) (layer "F.Cu") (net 12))
 (segment (start 71.2 58.34) (end 83.82 58.34) (width 0.4) (layer "F.Cu") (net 12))
 (via (at 71.12 58.42) (size 1.4) (drill 0.8) (layers "F.Cu" "B.Cu") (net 12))
 (via (at 45.72 58.42) (size 1.4) (drill 0.8) (layers "F.Cu" "B.Cu") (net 12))
 (segment (start 45.72 58.42) (end 71.12 58.42) (width 0.4) (layer "B.Cu") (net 12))
 (segment (start 33.02 38.1) (end 33.02 37.52) (width 0.8) (layer "F.Cu") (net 31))
 (segment (start 33.02 37.52) (end 32.68 37.52) (width 0.8) (layer "F.Cu") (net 31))
 (segment (start 32.48 38.1) (end 33.06 37.52) (width 0.8) (layer "F.Cu") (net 31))
 (segment (start 32.1 38.1) (end 33.02 38.1) (width 0.8) (layer "F.Cu") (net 31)))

